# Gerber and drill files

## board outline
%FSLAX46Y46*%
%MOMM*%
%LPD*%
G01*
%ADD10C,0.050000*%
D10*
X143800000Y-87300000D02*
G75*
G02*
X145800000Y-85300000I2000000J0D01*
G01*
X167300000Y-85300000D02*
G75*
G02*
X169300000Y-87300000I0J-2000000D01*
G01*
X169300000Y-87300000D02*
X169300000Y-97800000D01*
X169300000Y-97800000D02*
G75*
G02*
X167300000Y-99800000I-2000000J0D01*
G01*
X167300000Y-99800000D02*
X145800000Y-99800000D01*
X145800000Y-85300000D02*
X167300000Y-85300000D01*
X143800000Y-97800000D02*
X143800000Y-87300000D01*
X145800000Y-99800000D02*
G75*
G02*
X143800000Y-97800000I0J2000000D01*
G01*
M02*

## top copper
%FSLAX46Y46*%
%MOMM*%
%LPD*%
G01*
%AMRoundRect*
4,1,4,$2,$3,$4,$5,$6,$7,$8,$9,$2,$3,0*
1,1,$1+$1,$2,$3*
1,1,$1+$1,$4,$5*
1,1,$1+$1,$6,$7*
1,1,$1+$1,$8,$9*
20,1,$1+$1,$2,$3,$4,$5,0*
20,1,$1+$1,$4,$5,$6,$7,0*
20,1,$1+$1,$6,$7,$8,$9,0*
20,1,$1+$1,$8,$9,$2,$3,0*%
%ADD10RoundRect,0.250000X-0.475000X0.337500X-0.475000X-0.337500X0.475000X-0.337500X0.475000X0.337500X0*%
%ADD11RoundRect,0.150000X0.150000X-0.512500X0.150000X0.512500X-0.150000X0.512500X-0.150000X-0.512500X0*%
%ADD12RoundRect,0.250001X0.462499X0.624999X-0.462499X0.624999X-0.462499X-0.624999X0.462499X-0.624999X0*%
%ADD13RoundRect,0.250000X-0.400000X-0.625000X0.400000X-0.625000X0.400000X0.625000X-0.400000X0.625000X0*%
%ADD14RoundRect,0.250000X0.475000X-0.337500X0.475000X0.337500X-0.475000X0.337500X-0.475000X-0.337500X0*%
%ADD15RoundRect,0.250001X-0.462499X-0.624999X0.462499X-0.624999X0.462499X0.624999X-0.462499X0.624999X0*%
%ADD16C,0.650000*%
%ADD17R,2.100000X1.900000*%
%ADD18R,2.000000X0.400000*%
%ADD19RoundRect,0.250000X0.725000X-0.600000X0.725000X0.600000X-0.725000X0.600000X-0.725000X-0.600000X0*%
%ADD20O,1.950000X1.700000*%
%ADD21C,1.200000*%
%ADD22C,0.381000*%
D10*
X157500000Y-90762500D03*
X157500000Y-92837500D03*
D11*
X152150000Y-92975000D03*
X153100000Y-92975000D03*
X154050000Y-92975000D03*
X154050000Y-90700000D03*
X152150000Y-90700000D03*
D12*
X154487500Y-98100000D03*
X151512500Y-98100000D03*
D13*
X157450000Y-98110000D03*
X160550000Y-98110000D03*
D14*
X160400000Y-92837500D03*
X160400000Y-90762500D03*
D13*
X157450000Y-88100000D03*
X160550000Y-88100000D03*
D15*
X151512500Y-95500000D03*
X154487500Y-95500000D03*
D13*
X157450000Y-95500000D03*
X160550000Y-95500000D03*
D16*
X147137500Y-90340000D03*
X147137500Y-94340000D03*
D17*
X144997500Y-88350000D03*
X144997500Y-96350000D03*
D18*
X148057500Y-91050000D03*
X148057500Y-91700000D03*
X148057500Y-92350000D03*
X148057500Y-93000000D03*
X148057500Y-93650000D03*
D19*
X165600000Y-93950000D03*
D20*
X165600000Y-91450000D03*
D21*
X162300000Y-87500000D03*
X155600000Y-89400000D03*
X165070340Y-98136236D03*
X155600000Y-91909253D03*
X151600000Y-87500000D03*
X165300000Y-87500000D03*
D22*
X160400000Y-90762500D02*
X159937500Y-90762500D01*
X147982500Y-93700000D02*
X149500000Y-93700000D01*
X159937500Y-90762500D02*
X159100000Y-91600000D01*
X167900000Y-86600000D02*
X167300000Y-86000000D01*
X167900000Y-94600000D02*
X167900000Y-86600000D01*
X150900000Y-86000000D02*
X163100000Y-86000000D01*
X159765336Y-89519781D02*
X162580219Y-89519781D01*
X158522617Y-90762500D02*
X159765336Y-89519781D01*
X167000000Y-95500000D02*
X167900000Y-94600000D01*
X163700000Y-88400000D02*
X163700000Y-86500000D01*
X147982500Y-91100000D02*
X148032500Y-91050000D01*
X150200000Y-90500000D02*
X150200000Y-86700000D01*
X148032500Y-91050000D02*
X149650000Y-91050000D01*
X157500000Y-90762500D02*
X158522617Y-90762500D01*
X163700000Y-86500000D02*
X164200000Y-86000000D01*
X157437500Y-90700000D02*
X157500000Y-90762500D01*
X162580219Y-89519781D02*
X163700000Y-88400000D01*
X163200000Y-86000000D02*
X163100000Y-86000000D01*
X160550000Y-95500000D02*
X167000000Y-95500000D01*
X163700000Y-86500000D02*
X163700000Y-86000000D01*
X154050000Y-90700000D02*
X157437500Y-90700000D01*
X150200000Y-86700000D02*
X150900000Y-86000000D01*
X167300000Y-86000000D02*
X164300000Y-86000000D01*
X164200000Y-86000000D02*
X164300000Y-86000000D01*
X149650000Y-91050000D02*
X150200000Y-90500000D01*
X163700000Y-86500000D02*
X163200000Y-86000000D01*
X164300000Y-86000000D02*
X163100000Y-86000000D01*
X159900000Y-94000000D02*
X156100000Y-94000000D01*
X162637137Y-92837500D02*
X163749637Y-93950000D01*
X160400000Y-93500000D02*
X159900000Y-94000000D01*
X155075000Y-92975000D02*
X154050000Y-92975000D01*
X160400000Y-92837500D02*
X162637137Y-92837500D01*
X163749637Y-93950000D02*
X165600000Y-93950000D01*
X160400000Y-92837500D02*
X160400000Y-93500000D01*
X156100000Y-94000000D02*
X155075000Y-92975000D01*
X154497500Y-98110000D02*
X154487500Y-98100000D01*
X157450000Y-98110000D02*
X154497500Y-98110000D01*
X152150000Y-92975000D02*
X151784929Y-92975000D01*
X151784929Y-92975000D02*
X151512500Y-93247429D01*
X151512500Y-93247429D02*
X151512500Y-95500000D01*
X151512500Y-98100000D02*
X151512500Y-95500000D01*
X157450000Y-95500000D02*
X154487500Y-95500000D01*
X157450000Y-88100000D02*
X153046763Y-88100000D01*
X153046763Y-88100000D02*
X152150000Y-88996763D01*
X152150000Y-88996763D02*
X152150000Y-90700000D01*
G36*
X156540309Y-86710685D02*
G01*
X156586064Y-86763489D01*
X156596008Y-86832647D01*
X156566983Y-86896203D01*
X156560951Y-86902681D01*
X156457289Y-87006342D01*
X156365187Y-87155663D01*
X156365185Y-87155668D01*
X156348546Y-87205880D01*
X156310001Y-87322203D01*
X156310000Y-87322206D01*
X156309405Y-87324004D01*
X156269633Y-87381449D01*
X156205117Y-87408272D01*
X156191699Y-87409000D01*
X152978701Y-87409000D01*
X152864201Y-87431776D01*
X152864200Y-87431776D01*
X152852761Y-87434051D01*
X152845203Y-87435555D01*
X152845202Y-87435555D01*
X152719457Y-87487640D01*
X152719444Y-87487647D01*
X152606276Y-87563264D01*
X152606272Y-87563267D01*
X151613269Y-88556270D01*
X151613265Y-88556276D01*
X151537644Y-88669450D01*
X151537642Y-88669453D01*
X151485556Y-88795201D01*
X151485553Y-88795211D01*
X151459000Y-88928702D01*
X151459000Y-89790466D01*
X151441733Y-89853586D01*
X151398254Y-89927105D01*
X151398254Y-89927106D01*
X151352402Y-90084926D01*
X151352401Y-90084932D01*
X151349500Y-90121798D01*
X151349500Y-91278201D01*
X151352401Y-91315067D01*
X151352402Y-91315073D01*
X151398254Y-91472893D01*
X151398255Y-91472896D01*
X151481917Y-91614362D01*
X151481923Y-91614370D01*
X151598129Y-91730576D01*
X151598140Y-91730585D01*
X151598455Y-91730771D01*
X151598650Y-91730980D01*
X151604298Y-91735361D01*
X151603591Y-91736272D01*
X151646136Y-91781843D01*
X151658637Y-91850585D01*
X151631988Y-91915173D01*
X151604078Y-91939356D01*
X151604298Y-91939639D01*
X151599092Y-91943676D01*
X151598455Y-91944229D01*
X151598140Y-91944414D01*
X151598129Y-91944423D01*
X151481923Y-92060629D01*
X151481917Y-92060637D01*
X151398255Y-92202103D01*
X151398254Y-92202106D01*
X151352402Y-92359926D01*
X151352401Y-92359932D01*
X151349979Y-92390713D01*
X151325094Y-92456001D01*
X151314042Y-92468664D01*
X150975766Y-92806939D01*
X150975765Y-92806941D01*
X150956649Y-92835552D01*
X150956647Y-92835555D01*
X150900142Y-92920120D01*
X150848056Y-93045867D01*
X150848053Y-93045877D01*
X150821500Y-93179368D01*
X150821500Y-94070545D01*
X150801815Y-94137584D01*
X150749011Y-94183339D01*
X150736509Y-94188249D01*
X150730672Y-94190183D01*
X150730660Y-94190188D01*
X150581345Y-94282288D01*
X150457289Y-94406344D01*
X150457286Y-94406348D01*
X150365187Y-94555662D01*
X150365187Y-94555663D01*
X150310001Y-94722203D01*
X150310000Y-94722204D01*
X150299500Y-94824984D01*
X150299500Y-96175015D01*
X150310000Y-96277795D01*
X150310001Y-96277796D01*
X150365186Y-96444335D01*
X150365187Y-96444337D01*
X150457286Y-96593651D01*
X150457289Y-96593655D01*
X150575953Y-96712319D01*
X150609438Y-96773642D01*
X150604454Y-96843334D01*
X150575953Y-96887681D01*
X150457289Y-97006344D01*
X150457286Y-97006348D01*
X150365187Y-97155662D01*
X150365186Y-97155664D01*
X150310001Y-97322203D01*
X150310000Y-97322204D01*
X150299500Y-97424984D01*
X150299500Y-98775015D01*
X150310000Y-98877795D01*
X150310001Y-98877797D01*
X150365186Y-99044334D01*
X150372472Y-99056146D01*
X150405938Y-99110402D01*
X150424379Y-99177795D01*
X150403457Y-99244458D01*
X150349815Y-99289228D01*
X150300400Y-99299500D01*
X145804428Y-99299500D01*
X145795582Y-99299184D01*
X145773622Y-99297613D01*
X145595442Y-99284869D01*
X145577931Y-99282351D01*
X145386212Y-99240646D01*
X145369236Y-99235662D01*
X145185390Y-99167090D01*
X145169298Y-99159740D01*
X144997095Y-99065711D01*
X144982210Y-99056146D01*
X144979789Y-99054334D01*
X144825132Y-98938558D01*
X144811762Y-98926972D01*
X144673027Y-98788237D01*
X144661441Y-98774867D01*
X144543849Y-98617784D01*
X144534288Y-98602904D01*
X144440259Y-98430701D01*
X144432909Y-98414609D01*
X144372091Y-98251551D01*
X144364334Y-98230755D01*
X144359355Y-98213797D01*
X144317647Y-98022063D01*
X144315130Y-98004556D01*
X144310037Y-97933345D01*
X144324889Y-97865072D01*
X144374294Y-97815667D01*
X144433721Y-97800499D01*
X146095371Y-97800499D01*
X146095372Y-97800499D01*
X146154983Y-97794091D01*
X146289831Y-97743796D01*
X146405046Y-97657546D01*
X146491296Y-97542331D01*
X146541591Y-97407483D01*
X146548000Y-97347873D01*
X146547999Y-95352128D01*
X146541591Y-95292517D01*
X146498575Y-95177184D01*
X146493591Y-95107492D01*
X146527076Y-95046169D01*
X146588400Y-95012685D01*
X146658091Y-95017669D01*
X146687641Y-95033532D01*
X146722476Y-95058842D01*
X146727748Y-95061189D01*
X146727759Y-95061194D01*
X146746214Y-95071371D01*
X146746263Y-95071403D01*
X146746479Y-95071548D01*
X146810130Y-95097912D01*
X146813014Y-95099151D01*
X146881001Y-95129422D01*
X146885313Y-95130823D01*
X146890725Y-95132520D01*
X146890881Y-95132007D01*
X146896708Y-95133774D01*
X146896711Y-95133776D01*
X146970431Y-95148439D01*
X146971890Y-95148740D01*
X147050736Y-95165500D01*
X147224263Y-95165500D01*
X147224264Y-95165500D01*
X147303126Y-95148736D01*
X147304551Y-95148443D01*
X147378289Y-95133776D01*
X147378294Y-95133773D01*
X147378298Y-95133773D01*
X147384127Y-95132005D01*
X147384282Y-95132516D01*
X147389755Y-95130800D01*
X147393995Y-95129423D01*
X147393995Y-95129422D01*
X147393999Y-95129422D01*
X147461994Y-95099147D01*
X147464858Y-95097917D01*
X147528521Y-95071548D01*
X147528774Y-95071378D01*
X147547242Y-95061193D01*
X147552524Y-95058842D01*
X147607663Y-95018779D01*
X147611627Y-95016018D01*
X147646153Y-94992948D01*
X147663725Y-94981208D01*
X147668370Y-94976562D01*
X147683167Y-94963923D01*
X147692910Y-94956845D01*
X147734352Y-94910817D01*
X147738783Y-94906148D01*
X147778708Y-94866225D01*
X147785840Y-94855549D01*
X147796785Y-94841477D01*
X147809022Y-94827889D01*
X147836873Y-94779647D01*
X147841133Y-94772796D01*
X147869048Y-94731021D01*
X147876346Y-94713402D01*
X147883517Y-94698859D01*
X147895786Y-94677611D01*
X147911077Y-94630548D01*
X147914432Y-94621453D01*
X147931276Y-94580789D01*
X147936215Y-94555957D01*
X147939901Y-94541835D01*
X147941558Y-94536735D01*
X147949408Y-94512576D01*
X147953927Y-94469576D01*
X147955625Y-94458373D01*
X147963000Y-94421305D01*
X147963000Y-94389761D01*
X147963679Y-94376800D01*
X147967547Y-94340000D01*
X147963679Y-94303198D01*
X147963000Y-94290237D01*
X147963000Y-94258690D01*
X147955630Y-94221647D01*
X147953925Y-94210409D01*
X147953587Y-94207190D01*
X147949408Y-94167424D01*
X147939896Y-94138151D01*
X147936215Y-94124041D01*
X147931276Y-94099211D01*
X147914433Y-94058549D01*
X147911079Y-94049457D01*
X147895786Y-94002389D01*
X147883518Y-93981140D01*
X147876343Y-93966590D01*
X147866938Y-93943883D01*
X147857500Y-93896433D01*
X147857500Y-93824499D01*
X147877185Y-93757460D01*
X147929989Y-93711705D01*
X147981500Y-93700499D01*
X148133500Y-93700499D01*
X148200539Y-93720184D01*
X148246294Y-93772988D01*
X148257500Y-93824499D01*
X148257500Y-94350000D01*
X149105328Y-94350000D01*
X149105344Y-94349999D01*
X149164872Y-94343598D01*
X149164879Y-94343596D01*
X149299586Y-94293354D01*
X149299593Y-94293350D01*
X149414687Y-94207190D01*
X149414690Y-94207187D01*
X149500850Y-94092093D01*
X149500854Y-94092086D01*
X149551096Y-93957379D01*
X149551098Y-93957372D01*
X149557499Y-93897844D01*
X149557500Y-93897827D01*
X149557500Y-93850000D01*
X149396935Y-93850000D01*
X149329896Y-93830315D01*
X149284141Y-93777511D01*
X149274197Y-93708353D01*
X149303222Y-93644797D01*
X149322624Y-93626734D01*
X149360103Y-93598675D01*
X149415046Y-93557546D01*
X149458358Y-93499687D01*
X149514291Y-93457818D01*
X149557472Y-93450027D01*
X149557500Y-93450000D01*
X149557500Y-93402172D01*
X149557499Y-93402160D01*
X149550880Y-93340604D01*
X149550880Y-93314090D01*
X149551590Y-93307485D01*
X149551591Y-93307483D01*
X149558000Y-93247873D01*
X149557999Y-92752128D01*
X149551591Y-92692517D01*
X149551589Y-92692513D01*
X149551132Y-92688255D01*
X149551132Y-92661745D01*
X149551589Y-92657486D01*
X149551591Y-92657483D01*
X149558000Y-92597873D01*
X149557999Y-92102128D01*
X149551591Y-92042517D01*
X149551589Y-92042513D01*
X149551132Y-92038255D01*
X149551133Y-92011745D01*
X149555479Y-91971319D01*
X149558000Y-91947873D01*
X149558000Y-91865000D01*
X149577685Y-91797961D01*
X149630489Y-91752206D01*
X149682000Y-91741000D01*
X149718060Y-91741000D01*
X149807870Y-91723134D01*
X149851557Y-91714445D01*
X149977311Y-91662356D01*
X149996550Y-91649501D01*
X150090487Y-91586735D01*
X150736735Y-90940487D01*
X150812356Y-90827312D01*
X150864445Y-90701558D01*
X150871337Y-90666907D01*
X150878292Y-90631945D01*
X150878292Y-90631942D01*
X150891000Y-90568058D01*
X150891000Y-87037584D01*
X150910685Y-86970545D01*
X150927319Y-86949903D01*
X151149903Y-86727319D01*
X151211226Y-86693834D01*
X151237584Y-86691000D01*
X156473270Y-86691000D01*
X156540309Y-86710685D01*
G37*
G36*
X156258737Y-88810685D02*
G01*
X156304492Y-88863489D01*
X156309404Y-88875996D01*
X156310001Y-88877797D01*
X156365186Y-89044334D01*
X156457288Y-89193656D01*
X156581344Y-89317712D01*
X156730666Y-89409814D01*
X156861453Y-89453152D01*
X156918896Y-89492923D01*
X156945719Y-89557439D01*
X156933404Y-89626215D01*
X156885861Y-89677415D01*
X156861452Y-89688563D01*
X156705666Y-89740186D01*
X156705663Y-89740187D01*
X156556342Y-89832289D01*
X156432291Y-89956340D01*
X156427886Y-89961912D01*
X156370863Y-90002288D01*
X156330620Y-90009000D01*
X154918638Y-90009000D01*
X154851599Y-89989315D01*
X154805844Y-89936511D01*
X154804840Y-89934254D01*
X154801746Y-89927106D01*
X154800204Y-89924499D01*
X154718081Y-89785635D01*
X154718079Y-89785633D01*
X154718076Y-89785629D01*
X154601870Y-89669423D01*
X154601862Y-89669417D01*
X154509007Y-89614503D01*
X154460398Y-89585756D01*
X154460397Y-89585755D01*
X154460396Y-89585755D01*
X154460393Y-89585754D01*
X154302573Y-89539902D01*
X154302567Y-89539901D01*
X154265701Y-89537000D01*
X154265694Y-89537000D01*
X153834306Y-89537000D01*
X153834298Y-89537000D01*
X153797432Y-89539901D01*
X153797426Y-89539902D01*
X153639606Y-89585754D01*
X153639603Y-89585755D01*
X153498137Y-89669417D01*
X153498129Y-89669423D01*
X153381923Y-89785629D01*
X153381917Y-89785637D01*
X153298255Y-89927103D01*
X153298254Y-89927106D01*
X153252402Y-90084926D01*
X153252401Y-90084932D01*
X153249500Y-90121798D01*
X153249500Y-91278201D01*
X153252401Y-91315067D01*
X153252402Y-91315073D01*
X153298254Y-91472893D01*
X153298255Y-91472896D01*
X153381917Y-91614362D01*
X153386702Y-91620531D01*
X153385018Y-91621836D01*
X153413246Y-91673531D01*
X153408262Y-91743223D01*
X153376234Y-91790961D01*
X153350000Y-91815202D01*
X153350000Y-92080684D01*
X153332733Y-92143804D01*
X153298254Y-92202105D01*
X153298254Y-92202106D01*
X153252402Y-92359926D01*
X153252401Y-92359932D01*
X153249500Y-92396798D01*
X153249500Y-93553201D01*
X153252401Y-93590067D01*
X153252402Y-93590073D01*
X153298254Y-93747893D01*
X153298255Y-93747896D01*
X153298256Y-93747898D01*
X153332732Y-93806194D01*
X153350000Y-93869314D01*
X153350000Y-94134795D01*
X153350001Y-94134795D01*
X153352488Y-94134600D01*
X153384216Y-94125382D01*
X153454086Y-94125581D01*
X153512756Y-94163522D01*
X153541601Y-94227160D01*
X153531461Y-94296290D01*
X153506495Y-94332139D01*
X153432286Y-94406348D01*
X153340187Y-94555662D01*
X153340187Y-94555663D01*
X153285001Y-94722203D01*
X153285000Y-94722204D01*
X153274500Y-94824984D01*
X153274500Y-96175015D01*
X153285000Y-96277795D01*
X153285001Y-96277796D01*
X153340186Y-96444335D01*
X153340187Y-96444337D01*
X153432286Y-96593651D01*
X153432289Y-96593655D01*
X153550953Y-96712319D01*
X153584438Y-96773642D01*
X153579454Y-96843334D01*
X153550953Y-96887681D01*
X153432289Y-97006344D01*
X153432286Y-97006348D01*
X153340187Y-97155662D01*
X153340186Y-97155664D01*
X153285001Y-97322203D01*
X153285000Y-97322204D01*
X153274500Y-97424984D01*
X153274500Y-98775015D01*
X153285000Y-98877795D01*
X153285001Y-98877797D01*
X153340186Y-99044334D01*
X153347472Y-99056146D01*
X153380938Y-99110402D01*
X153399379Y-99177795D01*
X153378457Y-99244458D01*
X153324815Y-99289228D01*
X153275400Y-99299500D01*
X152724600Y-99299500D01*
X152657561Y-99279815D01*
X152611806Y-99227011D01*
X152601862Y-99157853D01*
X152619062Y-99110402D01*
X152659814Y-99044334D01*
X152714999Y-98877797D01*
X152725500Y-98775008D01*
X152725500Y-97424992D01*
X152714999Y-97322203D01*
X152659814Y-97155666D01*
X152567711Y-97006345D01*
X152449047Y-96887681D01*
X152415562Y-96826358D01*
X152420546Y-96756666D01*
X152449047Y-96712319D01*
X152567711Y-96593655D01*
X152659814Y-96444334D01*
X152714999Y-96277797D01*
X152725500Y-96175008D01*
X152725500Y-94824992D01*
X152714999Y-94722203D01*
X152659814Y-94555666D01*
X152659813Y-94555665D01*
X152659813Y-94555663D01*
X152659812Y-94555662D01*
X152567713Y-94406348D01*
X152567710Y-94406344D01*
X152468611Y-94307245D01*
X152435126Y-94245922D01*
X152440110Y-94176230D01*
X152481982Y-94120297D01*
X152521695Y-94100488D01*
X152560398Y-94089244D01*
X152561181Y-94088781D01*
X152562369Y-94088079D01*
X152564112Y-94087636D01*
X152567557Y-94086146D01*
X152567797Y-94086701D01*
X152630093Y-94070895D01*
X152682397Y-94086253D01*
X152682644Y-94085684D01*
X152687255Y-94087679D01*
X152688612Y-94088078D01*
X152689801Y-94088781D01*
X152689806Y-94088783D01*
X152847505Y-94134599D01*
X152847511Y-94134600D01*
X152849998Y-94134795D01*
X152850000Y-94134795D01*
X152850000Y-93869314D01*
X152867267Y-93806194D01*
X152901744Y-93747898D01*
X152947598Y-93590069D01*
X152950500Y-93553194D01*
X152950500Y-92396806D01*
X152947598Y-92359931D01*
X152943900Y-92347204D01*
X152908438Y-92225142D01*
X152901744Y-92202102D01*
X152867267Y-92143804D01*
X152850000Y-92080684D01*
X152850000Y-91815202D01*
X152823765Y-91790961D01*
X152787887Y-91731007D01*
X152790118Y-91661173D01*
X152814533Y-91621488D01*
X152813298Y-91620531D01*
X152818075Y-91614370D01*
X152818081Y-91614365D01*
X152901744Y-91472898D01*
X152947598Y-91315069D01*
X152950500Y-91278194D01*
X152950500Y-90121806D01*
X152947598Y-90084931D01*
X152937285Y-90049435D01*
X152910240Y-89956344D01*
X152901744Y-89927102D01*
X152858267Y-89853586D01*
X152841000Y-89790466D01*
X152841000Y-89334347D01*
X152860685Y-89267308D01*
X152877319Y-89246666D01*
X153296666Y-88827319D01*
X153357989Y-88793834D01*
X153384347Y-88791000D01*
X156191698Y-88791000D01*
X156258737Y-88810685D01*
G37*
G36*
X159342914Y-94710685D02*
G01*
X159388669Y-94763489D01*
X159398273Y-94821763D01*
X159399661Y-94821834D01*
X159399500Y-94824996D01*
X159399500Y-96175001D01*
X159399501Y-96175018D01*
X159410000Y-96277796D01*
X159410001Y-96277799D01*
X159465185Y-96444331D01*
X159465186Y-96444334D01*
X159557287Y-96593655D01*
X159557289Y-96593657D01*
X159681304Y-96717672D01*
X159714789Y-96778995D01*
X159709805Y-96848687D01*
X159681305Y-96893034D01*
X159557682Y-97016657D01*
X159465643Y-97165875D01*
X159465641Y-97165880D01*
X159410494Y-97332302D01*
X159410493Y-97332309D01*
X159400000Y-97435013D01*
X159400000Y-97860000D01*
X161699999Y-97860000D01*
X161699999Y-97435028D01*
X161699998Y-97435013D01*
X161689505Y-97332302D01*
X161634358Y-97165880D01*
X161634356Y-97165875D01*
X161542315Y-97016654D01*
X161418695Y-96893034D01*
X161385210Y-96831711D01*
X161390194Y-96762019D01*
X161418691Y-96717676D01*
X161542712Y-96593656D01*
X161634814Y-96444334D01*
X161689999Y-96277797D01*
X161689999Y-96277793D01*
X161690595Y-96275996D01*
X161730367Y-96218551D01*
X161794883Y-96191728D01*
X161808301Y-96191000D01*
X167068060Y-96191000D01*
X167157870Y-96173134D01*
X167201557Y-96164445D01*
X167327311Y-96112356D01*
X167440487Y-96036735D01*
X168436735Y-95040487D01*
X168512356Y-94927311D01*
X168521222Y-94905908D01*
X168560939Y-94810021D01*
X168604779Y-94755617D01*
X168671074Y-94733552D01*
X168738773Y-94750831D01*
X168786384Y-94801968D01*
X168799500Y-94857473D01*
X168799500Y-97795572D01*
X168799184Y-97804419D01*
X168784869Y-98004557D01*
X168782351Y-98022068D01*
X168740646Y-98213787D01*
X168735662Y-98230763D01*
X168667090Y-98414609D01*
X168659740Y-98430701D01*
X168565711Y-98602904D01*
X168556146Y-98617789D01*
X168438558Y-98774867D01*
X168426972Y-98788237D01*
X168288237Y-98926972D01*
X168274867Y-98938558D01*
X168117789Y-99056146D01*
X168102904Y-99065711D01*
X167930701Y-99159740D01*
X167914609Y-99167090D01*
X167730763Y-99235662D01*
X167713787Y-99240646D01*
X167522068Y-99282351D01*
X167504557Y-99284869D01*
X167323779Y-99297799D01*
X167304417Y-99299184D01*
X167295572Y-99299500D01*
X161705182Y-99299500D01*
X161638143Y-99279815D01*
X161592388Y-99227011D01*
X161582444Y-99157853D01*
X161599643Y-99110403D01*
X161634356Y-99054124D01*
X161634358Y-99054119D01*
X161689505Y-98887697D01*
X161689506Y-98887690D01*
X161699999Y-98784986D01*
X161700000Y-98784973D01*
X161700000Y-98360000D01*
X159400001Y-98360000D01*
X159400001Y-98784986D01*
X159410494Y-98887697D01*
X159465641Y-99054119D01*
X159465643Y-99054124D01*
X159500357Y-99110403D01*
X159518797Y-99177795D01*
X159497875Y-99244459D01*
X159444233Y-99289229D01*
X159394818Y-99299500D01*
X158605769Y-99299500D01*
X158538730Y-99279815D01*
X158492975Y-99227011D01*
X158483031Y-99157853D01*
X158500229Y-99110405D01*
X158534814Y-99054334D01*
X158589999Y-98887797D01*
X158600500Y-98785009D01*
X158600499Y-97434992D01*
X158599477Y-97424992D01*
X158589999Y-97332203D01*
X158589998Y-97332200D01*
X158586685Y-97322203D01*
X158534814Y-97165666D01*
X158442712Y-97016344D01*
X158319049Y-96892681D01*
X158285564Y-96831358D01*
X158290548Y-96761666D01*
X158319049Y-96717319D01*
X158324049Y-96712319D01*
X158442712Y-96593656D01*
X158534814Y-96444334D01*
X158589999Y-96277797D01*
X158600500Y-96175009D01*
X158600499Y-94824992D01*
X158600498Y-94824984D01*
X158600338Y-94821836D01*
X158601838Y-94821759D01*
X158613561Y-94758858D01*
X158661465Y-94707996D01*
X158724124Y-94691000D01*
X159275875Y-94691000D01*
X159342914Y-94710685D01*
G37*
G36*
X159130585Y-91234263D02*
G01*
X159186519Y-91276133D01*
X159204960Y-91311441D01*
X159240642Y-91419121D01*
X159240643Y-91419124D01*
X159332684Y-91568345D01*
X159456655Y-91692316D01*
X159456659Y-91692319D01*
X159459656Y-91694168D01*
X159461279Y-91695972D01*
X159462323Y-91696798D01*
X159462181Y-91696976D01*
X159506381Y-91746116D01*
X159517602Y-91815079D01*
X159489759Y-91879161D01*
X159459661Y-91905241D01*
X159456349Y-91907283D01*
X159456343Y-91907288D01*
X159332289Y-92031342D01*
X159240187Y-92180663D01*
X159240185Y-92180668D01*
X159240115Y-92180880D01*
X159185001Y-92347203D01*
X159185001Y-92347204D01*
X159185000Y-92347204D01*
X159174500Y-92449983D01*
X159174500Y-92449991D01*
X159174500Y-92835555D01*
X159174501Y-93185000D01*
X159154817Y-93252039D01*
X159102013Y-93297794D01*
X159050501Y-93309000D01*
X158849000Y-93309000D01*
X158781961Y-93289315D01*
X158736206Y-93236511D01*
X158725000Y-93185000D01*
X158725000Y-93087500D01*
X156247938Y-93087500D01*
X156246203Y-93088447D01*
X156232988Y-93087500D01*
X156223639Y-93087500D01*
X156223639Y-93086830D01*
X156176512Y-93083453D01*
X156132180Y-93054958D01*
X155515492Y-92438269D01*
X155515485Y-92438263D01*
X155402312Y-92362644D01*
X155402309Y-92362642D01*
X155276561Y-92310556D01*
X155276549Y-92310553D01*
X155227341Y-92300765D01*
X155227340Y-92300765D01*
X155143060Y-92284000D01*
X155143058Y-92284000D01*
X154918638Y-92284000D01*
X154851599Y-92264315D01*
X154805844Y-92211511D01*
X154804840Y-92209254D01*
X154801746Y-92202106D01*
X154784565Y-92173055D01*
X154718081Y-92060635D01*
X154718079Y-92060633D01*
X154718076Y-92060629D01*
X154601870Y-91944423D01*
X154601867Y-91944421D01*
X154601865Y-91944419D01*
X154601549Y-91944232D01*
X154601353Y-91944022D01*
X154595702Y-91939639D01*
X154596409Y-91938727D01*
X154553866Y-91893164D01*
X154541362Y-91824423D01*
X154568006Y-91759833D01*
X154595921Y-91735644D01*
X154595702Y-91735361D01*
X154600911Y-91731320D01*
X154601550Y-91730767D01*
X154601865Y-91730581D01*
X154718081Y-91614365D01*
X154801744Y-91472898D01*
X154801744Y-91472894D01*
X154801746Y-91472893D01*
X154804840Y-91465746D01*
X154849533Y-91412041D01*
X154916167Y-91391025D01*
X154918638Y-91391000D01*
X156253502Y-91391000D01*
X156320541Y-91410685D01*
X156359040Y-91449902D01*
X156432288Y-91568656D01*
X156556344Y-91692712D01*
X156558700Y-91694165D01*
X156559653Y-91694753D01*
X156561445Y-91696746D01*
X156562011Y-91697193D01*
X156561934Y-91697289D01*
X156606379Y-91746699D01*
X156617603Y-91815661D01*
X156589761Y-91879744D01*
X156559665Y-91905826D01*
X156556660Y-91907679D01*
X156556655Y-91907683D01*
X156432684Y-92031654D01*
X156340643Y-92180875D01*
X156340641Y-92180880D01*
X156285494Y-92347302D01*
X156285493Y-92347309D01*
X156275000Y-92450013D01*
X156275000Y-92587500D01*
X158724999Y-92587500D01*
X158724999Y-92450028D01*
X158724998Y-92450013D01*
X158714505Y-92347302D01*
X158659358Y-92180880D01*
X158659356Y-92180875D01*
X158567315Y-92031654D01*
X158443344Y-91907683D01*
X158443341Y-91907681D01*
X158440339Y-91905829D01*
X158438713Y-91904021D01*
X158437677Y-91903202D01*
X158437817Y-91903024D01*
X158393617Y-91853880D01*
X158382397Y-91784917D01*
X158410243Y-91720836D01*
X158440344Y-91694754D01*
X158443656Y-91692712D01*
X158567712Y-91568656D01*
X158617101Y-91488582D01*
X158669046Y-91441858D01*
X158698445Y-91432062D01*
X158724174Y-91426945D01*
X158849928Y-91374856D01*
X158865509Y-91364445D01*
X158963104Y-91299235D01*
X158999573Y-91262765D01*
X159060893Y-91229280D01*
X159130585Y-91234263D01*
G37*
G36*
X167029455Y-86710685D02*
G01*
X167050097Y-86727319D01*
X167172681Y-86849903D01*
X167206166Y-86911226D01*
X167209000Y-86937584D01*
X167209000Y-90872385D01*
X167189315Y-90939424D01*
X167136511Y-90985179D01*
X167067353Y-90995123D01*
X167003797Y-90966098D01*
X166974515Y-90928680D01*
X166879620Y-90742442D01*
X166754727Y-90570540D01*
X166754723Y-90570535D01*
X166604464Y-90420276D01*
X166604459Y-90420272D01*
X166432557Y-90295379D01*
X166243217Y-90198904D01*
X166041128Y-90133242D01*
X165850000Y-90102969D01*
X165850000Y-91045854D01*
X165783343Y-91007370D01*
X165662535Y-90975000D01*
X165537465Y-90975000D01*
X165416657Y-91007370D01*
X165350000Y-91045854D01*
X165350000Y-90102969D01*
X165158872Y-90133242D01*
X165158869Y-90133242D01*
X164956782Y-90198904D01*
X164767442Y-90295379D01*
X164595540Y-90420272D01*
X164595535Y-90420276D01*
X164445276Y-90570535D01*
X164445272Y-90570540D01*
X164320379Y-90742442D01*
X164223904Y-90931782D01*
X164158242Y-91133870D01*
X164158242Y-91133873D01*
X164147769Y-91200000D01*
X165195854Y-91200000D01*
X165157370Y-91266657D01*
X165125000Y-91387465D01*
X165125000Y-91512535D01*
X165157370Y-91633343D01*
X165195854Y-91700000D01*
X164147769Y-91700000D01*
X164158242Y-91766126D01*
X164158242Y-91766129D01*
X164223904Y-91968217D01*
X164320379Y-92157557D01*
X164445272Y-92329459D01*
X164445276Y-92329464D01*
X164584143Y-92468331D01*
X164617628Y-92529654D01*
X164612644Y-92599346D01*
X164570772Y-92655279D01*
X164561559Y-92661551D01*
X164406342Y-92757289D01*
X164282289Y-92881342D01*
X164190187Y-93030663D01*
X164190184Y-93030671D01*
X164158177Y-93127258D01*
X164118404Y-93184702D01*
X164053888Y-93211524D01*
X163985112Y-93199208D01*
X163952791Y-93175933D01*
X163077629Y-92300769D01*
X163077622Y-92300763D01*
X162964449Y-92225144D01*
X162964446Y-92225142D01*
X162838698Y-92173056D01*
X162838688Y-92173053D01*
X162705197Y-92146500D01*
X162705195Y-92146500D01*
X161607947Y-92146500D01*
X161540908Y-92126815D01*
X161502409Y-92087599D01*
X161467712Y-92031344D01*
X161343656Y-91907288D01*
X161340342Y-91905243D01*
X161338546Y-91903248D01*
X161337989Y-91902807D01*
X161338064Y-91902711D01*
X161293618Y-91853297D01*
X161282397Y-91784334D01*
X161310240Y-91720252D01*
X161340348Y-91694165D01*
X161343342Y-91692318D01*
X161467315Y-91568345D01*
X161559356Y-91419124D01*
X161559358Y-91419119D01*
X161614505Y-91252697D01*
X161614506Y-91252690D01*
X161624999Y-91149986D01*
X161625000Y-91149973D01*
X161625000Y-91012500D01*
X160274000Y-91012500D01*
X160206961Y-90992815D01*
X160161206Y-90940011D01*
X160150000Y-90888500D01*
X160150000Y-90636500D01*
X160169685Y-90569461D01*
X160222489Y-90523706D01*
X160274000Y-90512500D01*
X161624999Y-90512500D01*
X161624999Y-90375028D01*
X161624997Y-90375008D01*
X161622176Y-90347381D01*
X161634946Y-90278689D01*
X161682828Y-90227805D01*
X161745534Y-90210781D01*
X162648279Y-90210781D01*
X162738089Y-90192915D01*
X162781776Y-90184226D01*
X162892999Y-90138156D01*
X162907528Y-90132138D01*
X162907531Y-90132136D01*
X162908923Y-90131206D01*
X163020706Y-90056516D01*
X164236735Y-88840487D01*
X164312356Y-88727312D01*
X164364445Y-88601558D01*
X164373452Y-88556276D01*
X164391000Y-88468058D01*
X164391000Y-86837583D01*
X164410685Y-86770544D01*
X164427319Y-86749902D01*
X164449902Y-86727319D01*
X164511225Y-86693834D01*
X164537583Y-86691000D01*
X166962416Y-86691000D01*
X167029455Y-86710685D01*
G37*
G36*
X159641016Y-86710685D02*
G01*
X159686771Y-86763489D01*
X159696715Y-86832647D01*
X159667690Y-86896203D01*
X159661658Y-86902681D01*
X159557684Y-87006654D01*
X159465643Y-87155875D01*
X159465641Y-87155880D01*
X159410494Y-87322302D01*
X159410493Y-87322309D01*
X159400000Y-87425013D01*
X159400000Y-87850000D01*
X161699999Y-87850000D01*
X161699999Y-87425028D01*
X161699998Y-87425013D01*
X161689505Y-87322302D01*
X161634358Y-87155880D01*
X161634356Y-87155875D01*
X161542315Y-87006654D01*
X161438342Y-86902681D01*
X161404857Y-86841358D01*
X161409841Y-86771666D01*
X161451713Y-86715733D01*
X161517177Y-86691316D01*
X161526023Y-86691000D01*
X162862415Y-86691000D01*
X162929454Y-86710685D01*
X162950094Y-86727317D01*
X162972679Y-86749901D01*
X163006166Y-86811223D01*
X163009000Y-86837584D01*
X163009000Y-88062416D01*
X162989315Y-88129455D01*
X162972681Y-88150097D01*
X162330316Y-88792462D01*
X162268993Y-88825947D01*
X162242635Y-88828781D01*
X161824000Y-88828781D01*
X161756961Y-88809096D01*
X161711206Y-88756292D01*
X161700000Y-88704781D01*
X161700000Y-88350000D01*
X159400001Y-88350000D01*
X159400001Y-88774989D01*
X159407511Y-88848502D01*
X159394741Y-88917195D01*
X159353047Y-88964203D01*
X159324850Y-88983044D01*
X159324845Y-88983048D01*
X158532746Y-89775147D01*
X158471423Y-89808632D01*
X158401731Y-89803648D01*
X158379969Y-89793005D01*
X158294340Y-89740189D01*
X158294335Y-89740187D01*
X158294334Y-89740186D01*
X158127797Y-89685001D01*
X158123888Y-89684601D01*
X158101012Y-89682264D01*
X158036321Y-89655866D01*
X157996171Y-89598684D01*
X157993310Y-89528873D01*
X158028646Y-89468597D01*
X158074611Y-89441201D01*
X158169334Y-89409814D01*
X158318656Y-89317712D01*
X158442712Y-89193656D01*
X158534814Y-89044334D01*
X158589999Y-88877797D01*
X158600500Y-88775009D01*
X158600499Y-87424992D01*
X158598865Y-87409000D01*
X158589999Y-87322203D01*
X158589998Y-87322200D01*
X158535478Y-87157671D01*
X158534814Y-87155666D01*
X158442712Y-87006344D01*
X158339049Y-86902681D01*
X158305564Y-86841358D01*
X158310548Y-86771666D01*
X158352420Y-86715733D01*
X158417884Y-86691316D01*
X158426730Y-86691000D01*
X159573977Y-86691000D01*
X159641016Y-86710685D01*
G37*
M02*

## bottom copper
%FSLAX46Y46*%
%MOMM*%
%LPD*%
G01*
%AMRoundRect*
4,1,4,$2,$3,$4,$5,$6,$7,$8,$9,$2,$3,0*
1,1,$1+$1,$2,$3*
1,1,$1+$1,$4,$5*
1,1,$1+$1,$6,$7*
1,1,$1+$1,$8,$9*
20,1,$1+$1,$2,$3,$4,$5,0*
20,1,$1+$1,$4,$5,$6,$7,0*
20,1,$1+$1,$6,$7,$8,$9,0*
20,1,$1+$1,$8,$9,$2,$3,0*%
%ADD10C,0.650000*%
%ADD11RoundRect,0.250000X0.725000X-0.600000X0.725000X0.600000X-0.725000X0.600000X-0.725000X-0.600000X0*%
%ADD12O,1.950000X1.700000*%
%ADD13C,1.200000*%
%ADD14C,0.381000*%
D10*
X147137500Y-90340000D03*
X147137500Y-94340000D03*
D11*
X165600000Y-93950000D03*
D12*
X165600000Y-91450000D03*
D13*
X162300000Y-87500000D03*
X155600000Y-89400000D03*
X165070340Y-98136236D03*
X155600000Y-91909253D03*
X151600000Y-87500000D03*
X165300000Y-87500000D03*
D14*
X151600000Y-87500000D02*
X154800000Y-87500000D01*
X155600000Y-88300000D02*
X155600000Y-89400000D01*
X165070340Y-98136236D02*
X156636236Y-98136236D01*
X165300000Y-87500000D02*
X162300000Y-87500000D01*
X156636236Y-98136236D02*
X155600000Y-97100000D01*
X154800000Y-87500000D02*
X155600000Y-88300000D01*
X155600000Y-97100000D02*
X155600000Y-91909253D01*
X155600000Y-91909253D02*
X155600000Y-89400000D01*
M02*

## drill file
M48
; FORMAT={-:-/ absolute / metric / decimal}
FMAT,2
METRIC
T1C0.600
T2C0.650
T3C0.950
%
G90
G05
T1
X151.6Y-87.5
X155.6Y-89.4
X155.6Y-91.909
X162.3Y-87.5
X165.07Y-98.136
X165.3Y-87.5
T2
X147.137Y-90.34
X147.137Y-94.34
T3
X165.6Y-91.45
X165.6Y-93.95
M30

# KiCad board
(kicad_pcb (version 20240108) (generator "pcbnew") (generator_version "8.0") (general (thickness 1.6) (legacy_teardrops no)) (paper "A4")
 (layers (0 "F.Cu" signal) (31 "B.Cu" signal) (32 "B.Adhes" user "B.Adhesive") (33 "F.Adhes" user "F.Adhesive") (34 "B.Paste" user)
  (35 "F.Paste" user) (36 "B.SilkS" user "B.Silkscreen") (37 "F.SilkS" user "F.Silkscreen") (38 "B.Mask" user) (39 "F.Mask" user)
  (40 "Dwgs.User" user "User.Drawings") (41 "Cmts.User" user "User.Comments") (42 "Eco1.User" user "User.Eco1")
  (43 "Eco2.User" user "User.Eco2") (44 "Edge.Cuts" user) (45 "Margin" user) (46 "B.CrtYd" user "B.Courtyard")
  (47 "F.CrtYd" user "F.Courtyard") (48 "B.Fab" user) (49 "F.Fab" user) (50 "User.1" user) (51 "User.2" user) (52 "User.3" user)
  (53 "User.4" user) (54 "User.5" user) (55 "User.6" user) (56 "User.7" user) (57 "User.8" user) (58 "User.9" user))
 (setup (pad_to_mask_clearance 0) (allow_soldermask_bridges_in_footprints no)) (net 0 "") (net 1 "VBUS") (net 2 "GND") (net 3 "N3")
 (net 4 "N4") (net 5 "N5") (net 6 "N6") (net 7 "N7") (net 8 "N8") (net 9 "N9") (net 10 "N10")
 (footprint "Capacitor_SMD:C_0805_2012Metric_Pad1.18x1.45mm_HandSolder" (layer "F.Cu") (at 157.5 91.8 -90)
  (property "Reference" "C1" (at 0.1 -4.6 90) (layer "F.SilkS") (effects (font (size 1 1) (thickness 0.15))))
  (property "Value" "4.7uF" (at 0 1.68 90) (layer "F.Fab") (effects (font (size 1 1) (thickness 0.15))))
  (pad "1" smd roundrect (at -1.0375 0 270) (size 1.175 1.45) (layers "F.Cu" "F.Paste" "F.Mask") (roundrect_rratio 0.212766) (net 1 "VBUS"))
  (pad "2" smd roundrect (at 1.0375 0 270) (size 1.175 1.45) (layers "F.Cu" "F.Paste" "F.Mask") (roundrect_rratio 0.212766) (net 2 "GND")))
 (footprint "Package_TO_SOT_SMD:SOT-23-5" (layer "F.Cu") (at 153.1 91.8375 90)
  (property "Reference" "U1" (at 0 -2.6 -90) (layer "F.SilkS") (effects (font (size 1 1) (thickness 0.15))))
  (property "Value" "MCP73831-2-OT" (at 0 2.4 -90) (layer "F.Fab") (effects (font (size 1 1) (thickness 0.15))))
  (pad "1" smd roundrect (at -1.1375 -0.95 90) (size 1.325 0.6) (layers "F.Cu" "F.Paste" "F.Mask") (roundrect_rratio 0.25) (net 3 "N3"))
  (pad "2" smd roundrect (at -1.1375 0 90) (size 1.325 0.6) (layers "F.Cu" "F.Paste" "F.Mask") (roundrect_rratio 0.25) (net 2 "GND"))
  (pad "3" smd roundrect (at -1.1375 0.95 90) (size 1.325 0.6) (layers "F.Cu" "F.Paste" "F.Mask") (roundrect_rratio 0.25) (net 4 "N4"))
  (pad "4" smd roundrect (at 1.1375 0.95 90) (size 1.325 0.6) (layers "F.Cu" "F.Paste" "F.Mask") (roundrect_rratio 0.25) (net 1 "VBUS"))
  (pad "5" smd roundrect (at 1.1375 -0.95 90) (size 1.325 0.6) (layers "F.Cu" "F.Paste" "F.Mask") (roundrect_rratio 0.25) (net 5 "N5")))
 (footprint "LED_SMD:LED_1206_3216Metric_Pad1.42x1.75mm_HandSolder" (layer "F.Cu") (at 153 98.1 180)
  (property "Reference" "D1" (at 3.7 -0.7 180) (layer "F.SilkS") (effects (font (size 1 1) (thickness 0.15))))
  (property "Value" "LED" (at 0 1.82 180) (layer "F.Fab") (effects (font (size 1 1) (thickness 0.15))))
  (pad "1" smd roundrect (at -1.4875 0 180) (size 1.425 1.75) (layers "F.Cu" "F.Paste" "F.Mask") (roundrect_rratio 0.175439) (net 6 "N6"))
  (pad "2" smd roundrect (at 1.4875 0 180) (size 1.425 1.75) (layers "F.Cu" "F.Paste" "F.Mask") (roundrect_rratio 0.175439) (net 3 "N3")))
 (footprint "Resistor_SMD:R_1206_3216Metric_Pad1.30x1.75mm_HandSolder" (layer "F.Cu") (at 159 98.11)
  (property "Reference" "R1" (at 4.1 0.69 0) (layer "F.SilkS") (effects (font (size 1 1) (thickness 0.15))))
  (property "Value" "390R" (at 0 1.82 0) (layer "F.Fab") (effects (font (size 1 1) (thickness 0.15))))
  (pad "1" smd roundrect (at -1.55 0) (size 1.3 1.75) (layers "F.Cu" "F.Paste" "F.Mask") (roundrect_rratio 0.192308) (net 6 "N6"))
  (pad "2" smd roundrect (at 1.55 0) (size 1.3 1.75) (layers "F.Cu" "F.Paste" "F.Mask") (roundrect_rratio 0.192308) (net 2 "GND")))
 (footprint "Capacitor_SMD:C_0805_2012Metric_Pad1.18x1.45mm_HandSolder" (layer "F.Cu") (at 160.4 91.8 90)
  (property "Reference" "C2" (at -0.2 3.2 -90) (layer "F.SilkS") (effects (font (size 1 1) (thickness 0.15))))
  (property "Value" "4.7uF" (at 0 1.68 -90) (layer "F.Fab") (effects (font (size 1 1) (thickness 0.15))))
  (pad "1" smd roundrect (at -1.0375 0 90) (size 1.175 1.45) (layers "F.Cu" "F.Paste" "F.Mask") (roundrect_rratio 0.212766) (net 4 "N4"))
  (pad "2" smd roundrect (at 1.0375 0 90) (size 1.175 1.45) (layers "F.Cu" "F.Paste" "F.Mask") (roundrect_rratio 0.212766) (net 2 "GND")))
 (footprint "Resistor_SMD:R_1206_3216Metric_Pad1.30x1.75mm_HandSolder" (layer "F.Cu") (at 159 88.1)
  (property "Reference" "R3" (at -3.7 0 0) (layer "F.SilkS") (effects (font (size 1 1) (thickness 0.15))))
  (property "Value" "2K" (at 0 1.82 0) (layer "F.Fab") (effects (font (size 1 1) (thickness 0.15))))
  (pad "1" smd roundrect (at -1.55 0) (size 1.3 1.75) (layers "F.Cu" "F.Paste" "F.Mask") (roundrect_rratio 0.192308) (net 5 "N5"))
  (pad "2" smd roundrect (at 1.55 0) (size 1.3 1.75) (layers "F.Cu" "F.Paste" "F.Mask") (roundrect_rratio 0.192308) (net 2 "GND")))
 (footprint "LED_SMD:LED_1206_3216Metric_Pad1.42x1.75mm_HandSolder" (layer "F.Cu") (at 153 95.5)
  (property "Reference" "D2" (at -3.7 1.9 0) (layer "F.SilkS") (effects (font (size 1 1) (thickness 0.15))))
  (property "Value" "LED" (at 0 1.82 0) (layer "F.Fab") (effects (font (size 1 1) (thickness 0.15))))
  (pad "1" smd roundrect (at -1.4875 0) (size 1.425 1.75) (layers "F.Cu" "F.Paste" "F.Mask") (roundrect_rratio 0.175439) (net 3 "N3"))
  (pad "2" smd roundrect (at 1.4875 0) (size 1.425 1.75) (layers "F.Cu" "F.Paste" "F.Mask") (roundrect_rratio 0.175439) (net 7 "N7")))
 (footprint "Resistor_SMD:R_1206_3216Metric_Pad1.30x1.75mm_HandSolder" (layer "F.Cu") (at 159 95.5)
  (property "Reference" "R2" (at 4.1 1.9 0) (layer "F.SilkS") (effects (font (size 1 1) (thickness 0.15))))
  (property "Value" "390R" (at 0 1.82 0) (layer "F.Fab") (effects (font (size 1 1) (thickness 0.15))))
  (pad "1" smd roundrect (at -1.55 0) (size 1.3 1.75) (layers "F.Cu" "F.Paste" "F.Mask") (roundrect_rratio 0.192308) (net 7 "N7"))
  (pad "2" smd roundrect (at 1.55 0) (size 1.3 1.75) (layers "F.Cu" "F.Paste" "F.Mask") (roundrect_rratio 0.192308) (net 1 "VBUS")))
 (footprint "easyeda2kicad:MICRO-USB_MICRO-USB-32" (layer "F.Cu") (at 146.5275 92.35 -90)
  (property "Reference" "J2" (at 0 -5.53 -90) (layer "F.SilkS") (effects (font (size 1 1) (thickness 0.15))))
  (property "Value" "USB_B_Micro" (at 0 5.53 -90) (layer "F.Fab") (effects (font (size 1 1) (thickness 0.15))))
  (pad "" thru_hole circle (at -2.01 -0.61 270) (size 0.65 0.65) (drill 0.65) (layers "*.Cu" "*.Mask") (remove_unused_layers no))
  (pad "" thru_hole circle (at 1.99 -0.61 270) (size 0.65 0.65) (drill 0.65) (layers "*.Cu" "*.Mask") (remove_unused_layers no))
  (pad "0" smd rect (at -4 1.53) (size 2.1 1.9) (layers "F.Cu" "F.Paste" "F.Mask"))
  (pad "0" smd rect (at 4 1.53) (size 2.1 1.9) (layers "F.Cu" "F.Paste" "F.Mask"))
  (pad "1" smd rect (at -1.3 -1.53 180) (size 2 0.4) (layers "F.Cu" "F.Paste" "F.Mask") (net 1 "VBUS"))
  (pad "2" smd rect (at -0.65 -1.53 180) (size 2 0.4) (layers "F.Cu" "F.Paste" "F.Mask") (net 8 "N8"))
  (pad "3" smd rect (at 0 -1.53 180) (size 2 0.4) (layers "F.Cu" "F.Paste" "F.Mask") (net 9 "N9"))
  (pad "4" smd rect (at 0.65 -1.53 180) (size 2 0.4) (layers "F.Cu" "F.Paste" "F.Mask") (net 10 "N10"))
  (pad "5" smd rect (at 1.3 -1.53 180) (size 2 0.4) (layers "F.Cu" "F.Paste" "F.Mask") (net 2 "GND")))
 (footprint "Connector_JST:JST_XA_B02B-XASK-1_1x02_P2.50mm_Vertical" (layer "B.Cu") (at 165.6 93.95 90)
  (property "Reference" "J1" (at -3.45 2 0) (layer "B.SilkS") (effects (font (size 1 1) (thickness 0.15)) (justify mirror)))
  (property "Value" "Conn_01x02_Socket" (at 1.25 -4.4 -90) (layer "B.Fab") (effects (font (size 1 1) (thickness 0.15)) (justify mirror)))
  (pad "1" thru_hole roundrect (at 0 0 90) (size 1.7 1.95) (drill 0.95) (layers "*.Cu" "*.Mask") (remove_unused_layers no)
   (roundrect_rratio 0.147059) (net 4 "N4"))
  (pad "2" thru_hole oval (at 2.5 0 90) (size 1.7 1.95) (drill 0.95) (layers "*.Cu" "*.Mask") (remove_unused_layers no) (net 2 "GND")))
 (gr_arc (start 143.8 87.3) (mid 144.385786 85.885786) (end 145.8 85.3) (stroke (width 0.05) (type default)) (layer "Edge.Cuts"))
 (gr_arc (start 167.3 85.3) (mid 168.714214 85.885786) (end 169.3 87.3) (stroke (width 0.05) (type default)) (layer "Edge.Cuts"))
 (gr_line (start 169.3 87.3) (end 169.3 97.8) (stroke (width 0.05) (type default)) (layer "Edge.Cuts"))
 (gr_arc (start 169.3 97.8) (mid 168.714214 99.214214) (end 167.3 99.8) (stroke (width 0.05) (type default)) (layer "Edge.Cuts"))
 (gr_line (start 167.3 99.8) (end 145.8 99.8) (stroke (width 0.05) (type default)) (layer "Edge.Cuts"))
 (gr_line (start 145.8 85.3) (end 167.3 85.3) (stroke (width 0.05) (type default)) (layer "Edge.Cuts"))
 (gr_line (start 143.8 97.8) (end 143.8 87.3) (stroke (width 0.05) (type default)) (layer "Edge.Cuts"))
 (gr_arc (start 145.8 99.8) (mid 144.385786 99.214214) (end 143.8 97.8) (stroke (width 0.05) (type default)) (layer "Edge.Cuts"))
 (segment (start 160.4 90.7625) (end 159.9375 90.7625) (width 0.381) (layer "F.Cu") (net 2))
 (segment (start 147.9825 93.7) (end 149.5 93.7) (width 0.381) (layer "F.Cu") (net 2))
 (segment (start 159.9375 90.7625) (end 159.1 91.6) (width 0.381) (layer "F.Cu") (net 2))
 (via (at 162.3 87.5) (size 1.2) (drill 0.6) (layers "F.Cu" "B.Cu") (free yes) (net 2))
 (via (at 155.6 89.4) (size 1.2) (drill 0.6) (layers "F.Cu" "B.Cu") (free yes) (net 2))
 (via (at 165.07034 98.136236) (size 1.2) (drill 0.6) (layers "F.Cu" "B.Cu") (free yes) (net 2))
 (via (at 155.6 91.909253) (size 1.2) (drill 0.6) (layers "F.Cu" "B.Cu") (free yes) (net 2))
 (via (at 151.6 87.5) (size 1.2) (drill 0.6) (layers "F.Cu" "B.Cu") (free yes) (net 2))
 (via (at 165.3 87.5) (size 1.2) (drill 0.6) (layers "F.Cu" "B.Cu") (free yes) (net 2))
 (segment (start 151.6 87.5) (end 154.8 87.5) (width 0.381) (layer "B.Cu") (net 2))
 (segment (start 155.6 88.3) (end 155.6 89.4) (width 0.381) (layer "B.Cu") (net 2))
 (segment (start 165.07034 98.136236) (end 156.636236 98.136236) (width 0.381) (layer "B.Cu") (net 2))
 (segment (start 165.3 87.5) (end 162.3 87.5) (width 0.381) (layer "B.Cu") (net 2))
 (segment (start 156.636236 98.136236) (end 155.6 97.1) (width 0.381) (layer "B.Cu") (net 2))
 (segment (start 154.8 87.5) (end 155.6 88.3) (width 0.381) (layer "B.Cu") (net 2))
 (segment (start 155.6 97.1) (end 155.6 91.909253) (width 0.381) (layer "B.Cu") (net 2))
 (segment (start 155.6 91.909253) (end 155.6 89.4) (width 0.381) (layer "B.Cu") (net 2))
 (segment (start 167.9 86.6) (end 167.3 86) (width 0.381) (layer "F.Cu") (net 1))
 (segment (start 167.9 94.6) (end 167.9 86.6) (width 0.381) (layer "F.Cu") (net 1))
 (segment (start 150.9 86) (end 163.1 86) (width 0.381) (layer "F.Cu") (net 1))
 (segment (start 159.765336 89.519781) (end 162.580219 89.519781) (width 0.381) (layer "F.Cu") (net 1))
 (segment (start 158.522617 90.7625) (end 159.765336 89.519781) (width 0.381) (layer "F.Cu") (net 1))
 (segment (start 167 95.5) (end 167.9 94.6) (width 0.381) (layer "F.Cu") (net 1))
 (segment (start 163.7 88.4) (end 163.7 86.5) (width 0.381) (layer "F.Cu") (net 1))
 (segment (start 147.9825 91.1) (end 148.0325 91.05) (width 0.381) (layer "F.Cu") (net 1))
 (segment (start 150.2 90.5) (end 150.2 86.7) (width 0.381) (layer "F.Cu") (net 1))
 (segment (start 148.0325 91.05) (end 149.65 91.05) (width 0.381) (layer "F.Cu") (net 1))
 (segment (start 157.5 90.7625) (end 158.522617 90.7625) (width 0.381) (layer "F.Cu") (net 1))
 (segment (start 163.7 86.5) (end 164.2 86) (width 0.381) (layer "F.Cu") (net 1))
 (segment (start 157.4375 90.7) (end 157.5 90.7625) (width 0.381) (layer "F.Cu") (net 1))
 (segment (start 162.580219 89.519781) (end 163.7 88.4) (width 0.381) (layer "F.Cu") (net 1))
 (segment (start 163.2 86) (end 163.1 86) (width 0.381) (layer "F.Cu") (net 1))
 (segment (start 160.55 95.5) (end 167 95.5) (width 0.381) (layer "F.Cu") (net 1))
 (segment (start 163.7 86.5) (end 163.7 86) (width 0.381) (layer "F.Cu") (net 1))
 (segment (start 154.05 90.7) (end 157.4375 90.7) (width 0.381) (layer "F.Cu") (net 1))
 (segment (start 150.2 86.7) (end 150.9 86) (width 0.381) (layer "F.Cu") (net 1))
 (segment (start 167.3 86) (end 164.3 86) (width 0.381) (layer "F.Cu") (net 1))
 (segment (start 164.2 86) (end 164.3 86) (width 0.381) (layer "F.Cu") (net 1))
 (segment (start 149.65 91.05) (end 150.2 90.5) (width 0.381) (layer "F.Cu") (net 1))
 (segment (start 163.7 86.5) (end 163.2 86) (width 0.381) (layer "F.Cu") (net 1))
 (segment (start 164.3 86) (end 163.1 86) (width 0.381) (layer "F.Cu") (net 1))
 (segment (start 159.9 94) (end 156.1 94) (width 0.381) (layer "F.Cu") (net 4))
 (segment (start 162.637137 92.8375) (end 163.749637 93.95) (width 0.381) (layer "F.Cu") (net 4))
 (segment (start 160.4 93.5) (end 159.9 94) (width 0.381) (layer "F.Cu") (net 4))
 (segment (start 155.075 92.975) (end 154.05 92.975) (width 0.381) (layer "F.Cu") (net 4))
 (segment (start 160.4 92.8375) (end 162.637137 92.8375) (width 0.381) (layer "F.Cu") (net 4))
 (segment (start 163.749637 93.95) (end 165.6 93.95) (width 0.381) (layer "F.Cu") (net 4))
 (segment (start 160.4 92.8375) (end 160.4 93.5) (width 0.381) (layer "F.Cu") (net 4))
 (segment (start 156.1 94) (end 155.075 92.975) (width 0.381) (layer "F.Cu") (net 4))
 (segment (start 154.4975 98.11) (end 154.4875 98.1) (width 0.381) (layer "F.Cu") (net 6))
 (segment (start 157.45 98.11) (end 154.4975 98.11) (width 0.381) (layer "F.Cu") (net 6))
 (segment (start 152.15 92.975) (end 151.784929 92.975) (width 0.381) (layer "F.Cu") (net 3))
 (segment (start 151.784929 92.975) (end 151.5125 93.247429) (width 0.381) (layer "F.Cu") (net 3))
 (segment (start 151.5125 93.247429) (end 151.5125 95.5) (width 0.381) (layer "F.Cu") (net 3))
 (segment (start 151.5125 98.1) (end 151.5125 95.5) (width 0.381) (layer "F.Cu") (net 3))
 (segment (start 157.45 95.5) (end 154.4875 95.5) (width 0.381) (layer "F.Cu") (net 7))
 (segment (start 157.45 88.1) (end 153.046763 88.1) (width 0.381) (layer "F.Cu") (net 5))
 (segment (start 153.046763 88.1) (end 152.15 88.996763) (width 0.381) (layer "F.Cu") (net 5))
 (segment (start 152.15 88.996763) (end 152.15 90.7) (width 0.381) (layer "F.Cu") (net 5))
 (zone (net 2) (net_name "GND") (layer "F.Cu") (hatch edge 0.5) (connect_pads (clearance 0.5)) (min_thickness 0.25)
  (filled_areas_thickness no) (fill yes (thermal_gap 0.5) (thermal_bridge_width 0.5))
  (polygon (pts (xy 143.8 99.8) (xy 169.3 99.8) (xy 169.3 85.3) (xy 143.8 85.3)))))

